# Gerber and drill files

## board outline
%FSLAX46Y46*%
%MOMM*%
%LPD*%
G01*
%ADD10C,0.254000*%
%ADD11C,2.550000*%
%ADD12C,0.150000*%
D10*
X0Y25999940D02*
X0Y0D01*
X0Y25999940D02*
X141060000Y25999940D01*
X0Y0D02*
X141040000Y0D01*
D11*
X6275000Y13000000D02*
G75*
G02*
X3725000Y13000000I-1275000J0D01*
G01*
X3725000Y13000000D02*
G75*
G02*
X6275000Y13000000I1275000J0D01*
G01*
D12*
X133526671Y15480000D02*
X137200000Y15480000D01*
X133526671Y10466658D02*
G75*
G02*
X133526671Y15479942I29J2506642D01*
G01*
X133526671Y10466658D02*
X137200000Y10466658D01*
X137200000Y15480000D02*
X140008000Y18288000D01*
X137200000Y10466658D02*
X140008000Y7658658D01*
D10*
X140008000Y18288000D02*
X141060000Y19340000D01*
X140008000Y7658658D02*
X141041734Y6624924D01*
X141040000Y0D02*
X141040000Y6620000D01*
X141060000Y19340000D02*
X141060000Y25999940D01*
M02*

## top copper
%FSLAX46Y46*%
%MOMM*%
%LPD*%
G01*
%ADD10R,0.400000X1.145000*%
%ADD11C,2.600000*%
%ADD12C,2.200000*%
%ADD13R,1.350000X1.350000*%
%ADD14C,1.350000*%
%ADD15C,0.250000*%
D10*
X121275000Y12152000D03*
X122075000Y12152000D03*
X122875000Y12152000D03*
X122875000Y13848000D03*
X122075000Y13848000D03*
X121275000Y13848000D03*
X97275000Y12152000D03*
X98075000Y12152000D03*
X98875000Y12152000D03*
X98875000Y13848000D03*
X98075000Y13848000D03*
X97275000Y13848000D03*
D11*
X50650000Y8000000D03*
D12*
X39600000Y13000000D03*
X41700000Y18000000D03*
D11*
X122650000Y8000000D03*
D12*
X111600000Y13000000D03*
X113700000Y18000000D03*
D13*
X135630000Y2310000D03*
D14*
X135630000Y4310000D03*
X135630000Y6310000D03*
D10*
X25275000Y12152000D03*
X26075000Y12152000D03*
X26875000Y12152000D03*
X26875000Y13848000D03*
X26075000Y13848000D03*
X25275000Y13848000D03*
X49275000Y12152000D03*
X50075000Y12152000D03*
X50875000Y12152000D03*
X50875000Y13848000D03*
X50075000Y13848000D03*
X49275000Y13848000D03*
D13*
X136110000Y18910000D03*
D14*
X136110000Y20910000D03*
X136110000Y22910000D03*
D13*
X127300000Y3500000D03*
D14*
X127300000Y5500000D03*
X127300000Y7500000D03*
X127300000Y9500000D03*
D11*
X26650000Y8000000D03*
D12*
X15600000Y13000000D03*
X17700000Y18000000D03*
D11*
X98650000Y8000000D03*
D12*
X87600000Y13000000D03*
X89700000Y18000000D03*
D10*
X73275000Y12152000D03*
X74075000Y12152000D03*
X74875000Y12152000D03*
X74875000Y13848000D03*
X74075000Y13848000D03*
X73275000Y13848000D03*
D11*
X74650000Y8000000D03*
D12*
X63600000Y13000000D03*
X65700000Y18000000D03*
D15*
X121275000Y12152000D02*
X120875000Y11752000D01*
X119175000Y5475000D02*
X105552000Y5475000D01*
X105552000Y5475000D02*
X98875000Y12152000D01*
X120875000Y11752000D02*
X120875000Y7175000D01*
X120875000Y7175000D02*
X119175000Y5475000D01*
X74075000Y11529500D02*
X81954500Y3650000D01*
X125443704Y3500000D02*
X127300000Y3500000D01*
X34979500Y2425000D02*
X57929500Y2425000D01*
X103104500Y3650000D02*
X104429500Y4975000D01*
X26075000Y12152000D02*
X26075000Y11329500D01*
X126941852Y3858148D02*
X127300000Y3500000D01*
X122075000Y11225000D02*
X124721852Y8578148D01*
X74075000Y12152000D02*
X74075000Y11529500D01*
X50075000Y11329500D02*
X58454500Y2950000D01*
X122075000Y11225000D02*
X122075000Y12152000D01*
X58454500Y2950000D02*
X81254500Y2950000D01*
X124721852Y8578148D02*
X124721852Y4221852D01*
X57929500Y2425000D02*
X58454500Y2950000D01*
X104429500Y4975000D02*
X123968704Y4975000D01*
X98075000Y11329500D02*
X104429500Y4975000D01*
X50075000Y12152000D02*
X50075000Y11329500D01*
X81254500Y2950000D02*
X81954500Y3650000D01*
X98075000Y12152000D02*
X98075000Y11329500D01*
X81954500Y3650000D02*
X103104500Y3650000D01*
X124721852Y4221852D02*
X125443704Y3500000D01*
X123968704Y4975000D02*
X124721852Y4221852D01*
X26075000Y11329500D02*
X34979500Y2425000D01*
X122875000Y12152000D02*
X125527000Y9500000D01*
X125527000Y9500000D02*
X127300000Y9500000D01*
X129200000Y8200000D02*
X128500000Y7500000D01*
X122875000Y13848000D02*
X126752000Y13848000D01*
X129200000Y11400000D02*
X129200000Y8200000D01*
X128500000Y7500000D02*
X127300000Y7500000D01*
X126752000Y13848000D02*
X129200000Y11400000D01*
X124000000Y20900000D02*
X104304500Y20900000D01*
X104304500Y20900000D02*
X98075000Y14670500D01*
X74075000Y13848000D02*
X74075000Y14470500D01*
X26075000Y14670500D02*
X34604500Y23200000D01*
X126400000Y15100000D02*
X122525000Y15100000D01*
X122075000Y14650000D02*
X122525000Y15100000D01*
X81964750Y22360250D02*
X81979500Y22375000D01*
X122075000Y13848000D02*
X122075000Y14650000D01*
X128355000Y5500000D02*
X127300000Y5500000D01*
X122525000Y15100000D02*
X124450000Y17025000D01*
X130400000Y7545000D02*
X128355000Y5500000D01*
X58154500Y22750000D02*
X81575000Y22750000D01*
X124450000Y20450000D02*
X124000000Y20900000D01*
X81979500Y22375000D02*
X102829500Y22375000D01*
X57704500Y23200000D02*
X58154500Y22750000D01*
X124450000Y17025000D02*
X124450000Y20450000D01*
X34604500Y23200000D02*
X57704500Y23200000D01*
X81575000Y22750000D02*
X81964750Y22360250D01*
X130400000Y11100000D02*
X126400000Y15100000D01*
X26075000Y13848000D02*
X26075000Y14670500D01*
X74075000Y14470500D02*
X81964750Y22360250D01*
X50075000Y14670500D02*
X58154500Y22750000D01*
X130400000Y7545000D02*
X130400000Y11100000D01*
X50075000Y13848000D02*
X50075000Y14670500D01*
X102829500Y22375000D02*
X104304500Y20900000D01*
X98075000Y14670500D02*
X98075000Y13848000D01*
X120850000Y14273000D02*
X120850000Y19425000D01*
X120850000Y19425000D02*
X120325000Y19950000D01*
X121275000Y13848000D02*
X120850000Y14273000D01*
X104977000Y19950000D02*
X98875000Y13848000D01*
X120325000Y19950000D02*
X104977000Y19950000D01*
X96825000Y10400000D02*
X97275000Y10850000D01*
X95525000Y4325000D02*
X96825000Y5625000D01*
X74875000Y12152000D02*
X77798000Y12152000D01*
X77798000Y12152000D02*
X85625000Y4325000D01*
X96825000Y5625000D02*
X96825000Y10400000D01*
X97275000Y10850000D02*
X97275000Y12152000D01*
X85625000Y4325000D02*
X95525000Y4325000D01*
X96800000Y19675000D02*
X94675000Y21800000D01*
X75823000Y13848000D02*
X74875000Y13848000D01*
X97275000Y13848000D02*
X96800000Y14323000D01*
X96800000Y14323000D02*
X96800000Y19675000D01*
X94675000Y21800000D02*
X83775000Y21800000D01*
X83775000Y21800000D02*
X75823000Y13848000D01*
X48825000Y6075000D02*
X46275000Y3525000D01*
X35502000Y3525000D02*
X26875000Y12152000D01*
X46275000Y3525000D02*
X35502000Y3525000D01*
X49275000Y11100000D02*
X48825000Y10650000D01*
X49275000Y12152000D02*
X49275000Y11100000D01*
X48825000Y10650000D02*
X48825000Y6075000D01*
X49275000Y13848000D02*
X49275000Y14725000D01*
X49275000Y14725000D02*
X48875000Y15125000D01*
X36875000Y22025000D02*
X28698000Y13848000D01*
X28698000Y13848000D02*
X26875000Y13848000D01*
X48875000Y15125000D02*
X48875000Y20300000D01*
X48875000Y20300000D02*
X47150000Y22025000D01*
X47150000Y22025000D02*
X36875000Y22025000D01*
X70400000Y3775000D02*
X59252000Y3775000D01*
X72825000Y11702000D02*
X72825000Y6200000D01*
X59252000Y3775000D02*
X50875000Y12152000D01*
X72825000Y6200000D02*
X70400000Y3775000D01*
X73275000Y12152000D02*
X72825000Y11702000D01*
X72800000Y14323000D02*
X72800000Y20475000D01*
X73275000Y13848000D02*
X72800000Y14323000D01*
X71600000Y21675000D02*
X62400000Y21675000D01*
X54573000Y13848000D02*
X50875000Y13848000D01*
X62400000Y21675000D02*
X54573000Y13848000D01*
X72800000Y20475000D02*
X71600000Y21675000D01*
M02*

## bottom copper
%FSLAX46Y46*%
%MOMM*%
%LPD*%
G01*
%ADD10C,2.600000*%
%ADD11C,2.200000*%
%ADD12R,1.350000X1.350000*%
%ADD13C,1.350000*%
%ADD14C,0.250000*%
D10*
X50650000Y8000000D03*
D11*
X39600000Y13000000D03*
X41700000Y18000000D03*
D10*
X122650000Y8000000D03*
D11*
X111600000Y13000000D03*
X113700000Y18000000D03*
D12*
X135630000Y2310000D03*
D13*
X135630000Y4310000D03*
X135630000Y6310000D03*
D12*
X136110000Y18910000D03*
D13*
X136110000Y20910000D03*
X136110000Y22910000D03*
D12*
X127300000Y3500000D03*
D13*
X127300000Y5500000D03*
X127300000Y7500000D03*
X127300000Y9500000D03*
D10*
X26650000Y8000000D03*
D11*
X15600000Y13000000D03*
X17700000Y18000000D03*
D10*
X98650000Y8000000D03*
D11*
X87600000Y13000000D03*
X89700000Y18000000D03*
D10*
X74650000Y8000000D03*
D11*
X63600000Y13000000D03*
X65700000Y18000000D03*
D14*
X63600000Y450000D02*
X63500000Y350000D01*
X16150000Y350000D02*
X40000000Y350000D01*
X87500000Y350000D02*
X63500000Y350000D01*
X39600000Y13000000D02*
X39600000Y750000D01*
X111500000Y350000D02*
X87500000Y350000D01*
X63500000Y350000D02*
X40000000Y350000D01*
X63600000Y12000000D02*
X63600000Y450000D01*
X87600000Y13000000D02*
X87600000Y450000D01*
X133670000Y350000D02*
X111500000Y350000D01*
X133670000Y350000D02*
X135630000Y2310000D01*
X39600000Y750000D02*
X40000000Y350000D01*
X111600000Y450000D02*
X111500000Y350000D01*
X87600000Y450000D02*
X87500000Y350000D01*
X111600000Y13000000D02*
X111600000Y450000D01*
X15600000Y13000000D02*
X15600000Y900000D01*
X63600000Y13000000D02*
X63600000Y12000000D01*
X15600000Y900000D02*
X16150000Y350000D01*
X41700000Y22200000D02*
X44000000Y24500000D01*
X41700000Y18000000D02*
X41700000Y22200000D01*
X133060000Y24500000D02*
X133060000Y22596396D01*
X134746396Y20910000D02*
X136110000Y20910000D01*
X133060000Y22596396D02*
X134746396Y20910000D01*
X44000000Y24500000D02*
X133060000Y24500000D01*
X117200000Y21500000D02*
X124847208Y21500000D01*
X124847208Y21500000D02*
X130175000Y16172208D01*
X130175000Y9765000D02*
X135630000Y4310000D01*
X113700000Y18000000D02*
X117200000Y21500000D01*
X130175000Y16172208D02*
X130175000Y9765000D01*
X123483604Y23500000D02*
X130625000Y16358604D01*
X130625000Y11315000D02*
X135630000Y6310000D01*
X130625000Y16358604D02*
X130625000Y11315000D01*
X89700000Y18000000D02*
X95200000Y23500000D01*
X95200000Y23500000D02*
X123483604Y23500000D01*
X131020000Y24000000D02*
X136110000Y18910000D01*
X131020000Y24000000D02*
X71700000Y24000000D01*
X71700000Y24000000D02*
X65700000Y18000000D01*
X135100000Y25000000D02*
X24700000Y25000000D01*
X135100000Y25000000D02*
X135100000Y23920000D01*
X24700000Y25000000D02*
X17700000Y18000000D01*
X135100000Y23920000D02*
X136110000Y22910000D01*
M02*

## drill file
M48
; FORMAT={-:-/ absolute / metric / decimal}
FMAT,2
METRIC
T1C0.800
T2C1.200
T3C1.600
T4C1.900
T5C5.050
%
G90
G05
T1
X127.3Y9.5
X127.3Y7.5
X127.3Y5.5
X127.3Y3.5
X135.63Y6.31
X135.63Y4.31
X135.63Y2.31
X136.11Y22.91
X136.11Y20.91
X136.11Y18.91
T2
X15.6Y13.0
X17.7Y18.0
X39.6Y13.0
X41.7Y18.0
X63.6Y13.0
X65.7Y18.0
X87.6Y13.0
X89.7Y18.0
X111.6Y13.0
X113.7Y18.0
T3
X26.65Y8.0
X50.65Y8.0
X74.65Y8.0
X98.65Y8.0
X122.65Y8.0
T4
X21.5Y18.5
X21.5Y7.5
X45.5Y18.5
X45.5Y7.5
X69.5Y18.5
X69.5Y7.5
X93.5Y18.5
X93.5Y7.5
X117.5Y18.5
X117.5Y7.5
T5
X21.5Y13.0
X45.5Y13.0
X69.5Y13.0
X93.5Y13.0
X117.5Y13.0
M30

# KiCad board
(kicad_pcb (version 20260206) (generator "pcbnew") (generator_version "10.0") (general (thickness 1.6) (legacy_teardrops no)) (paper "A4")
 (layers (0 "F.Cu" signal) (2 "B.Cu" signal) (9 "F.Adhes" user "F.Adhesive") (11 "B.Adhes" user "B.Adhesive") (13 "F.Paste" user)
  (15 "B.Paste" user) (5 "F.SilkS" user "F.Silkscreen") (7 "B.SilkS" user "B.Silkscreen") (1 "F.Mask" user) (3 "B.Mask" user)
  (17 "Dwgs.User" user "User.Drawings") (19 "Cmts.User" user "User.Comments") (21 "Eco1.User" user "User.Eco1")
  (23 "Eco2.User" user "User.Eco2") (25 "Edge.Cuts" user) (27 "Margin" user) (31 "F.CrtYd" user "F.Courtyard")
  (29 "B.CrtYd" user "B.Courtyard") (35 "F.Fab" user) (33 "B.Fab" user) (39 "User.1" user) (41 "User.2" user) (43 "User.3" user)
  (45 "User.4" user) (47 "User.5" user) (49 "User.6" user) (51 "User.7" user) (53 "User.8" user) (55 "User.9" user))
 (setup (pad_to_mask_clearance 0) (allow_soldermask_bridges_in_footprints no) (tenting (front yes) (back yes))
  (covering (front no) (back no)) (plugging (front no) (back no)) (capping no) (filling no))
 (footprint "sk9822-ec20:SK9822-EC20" (layer "F.Cu") (at 122.075 -13 90)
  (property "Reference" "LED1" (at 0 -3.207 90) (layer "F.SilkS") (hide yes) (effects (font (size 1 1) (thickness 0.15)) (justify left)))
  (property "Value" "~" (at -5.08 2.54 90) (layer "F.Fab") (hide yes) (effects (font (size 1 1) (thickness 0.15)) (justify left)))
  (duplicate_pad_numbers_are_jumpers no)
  (pad "1" smd rect (at -0.848 -0.8 90) (size 1.145 0.4) (layers "F.Cu" "F.Mask" "F.Paste") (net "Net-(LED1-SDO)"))
  (pad "2" smd rect (at -0.848 0 90) (size 1.145 0.4) (layers "F.Cu" "F.Mask" "F.Paste") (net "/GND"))
  (pad "3" smd rect (at -0.848 0.8 90) (size 1.145 0.4) (layers "F.Cu" "F.Mask" "F.Paste") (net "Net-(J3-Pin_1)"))
  (pad "4" smd rect (at 0.848 0.8 90) (size 1.145 0.4) (layers "F.Cu" "F.Mask" "F.Paste") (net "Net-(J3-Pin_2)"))
  (pad "5" smd rect (at 0.848 0 90) (size 1.145 0.4) (layers "F.Cu" "F.Mask" "F.Paste") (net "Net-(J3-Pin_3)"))
  (pad "6" smd rect (at 0.848 -0.8 90) (size 1.145 0.4) (layers "F.Cu" "F.Mask" "F.Paste") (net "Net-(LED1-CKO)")))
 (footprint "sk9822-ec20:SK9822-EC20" (layer "F.Cu") (at 98.075 -13 90)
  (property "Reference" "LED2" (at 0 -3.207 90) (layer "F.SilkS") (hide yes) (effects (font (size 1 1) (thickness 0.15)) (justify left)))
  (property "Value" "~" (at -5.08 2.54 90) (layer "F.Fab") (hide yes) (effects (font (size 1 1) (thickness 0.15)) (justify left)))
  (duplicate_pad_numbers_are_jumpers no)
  (pad "1" smd rect (at -0.848 -0.8 90) (size 1.145 0.4) (layers "F.Cu" "F.Mask" "F.Paste") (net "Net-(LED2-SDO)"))
  (pad "2" smd rect (at -0.848 0 90) (size 1.145 0.4) (layers "F.Cu" "F.Mask" "F.Paste") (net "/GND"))
  (pad "3" smd rect (at -0.848 0.8 90) (size 1.145 0.4) (layers "F.Cu" "F.Mask" "F.Paste") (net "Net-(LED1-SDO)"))
  (pad "4" smd rect (at 0.848 0.8 90) (size 1.145 0.4) (layers "F.Cu" "F.Mask" "F.Paste") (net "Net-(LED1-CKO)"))
  (pad "5" smd rect (at 0.848 0 90) (size 1.145 0.4) (layers "F.Cu" "F.Mask" "F.Paste") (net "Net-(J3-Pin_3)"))
  (pad "6" smd rect (at 0.848 -0.8 90) (size 1.145 0.4) (layers "F.Cu" "F.Mask" "F.Paste") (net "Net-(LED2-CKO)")))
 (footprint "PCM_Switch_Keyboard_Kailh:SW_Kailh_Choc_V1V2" (layer "F.Cu") (at 45.5 -13 90)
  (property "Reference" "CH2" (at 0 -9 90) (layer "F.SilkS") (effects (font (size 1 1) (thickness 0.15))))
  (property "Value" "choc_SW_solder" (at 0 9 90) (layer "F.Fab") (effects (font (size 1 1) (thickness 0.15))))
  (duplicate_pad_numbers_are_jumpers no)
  (pad "" np_thru_hole circle (at -5.5 0 90) (size 1.9 1.9) (drill 1.9) (layers "*.Cu" "*.Mask"))
  (pad "" thru_hole circle (at -5 5.15 90) (size 2.6 2.6) (drill 1.6) (layers "*.Cu" "*.Mask") (remove_unused_layers no)
   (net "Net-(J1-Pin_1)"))
  (pad "" np_thru_hole circle (at 0 0 90) (size 5.05 5.05) (drill 5.05) (layers "*.Cu" "*.Mask"))
  (pad "" np_thru_hole circle (at 5.5 0 90) (size 1.9 1.9) (drill 1.9) (layers "*.Cu" "*.Mask"))
  (pad "1" thru_hole circle (at 0 -5.9 90) (size 2.2 2.2) (drill 1.2) (layers "*.Cu" "*.Mask") (remove_unused_layers no)
   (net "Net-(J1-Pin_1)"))
  (pad "2" thru_hole circle (at 5 -3.8 90) (size 2.2 2.2) (drill 1.2) (layers "*.Cu" "*.Mask") (remove_unused_layers no)
   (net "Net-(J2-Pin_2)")))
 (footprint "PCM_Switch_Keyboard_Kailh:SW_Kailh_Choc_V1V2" (layer "F.Cu") (at 117.5 -13 90)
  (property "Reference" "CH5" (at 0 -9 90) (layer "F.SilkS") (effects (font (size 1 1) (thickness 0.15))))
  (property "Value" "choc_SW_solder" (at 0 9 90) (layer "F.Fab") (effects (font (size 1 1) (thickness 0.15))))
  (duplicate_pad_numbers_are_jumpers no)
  (pad "" np_thru_hole circle (at -5.5 0 90) (size 1.9 1.9) (drill 1.9) (layers "*.Cu" "*.Mask"))
  (pad "" thru_hole circle (at -5 5.15 90) (size 2.6 2.6) (drill 1.6) (layers "*.Cu" "*.Mask") (remove_unused_layers no)
   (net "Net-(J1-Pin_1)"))
  (pad "" np_thru_hole circle (at 0 0 90) (size 5.05 5.05) (drill 5.05) (layers "*.Cu" "*.Mask"))
  (pad "" np_thru_hole circle (at 5.5 0 90) (size 1.9 1.9) (drill 1.9) (layers "*.Cu" "*.Mask"))
  (pad "1" thru_hole circle (at 0 -5.9 90) (size 2.2 2.2) (drill 1.2) (layers "*.Cu" "*.Mask") (remove_unused_layers no)
   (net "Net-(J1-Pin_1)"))
  (pad "2" thru_hole circle (at 5 -3.8 90) (size 2.2 2.2) (drill 1.2) (layers "*.Cu" "*.Mask") (remove_unused_layers no)
   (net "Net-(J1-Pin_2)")))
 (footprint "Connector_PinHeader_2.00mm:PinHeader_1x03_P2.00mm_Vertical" (layer "F.Cu") (at 135.63 -2.31 180)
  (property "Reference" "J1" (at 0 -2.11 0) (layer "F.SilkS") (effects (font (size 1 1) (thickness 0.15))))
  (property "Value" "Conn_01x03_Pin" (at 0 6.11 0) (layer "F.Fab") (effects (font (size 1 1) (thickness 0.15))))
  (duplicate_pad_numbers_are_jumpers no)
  (pad "1" thru_hole rect (at 0 0 180) (size 1.35 1.35) (drill 0.8) (layers "*.Cu" "*.Mask") (remove_unused_layers no)
   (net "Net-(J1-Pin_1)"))
  (pad "2" thru_hole circle (at 0 2 180) (size 1.35 1.35) (drill 0.8) (layers "*.Cu" "*.Mask") (remove_unused_layers no)
   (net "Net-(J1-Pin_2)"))
  (pad "3" thru_hole circle (at 0 4 180) (size 1.35 1.35) (drill 0.8) (layers "*.Cu" "*.Mask") (remove_unused_layers no)
   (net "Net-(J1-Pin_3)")))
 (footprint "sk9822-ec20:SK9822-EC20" (layer "F.Cu") (at 26.075 -13 90)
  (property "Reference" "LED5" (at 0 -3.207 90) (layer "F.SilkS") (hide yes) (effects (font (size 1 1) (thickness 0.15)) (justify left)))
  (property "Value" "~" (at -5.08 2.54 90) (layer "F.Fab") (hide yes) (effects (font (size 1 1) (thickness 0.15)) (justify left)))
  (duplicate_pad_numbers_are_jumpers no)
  (pad "1" smd rect (at -0.848 -0.8 90) (size 1.145 0.4) (layers "F.Cu" "F.Mask" "F.Paste") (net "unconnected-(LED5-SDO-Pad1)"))
  (pad "2" smd rect (at -0.848 0 90) (size 1.145 0.4) (layers "F.Cu" "F.Mask" "F.Paste") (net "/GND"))
  (pad "3" smd rect (at -0.848 0.8 90) (size 1.145 0.4) (layers "F.Cu" "F.Mask" "F.Paste") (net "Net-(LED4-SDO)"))
  (pad "4" smd rect (at 0.848 0.8 90) (size 1.145 0.4) (layers "F.Cu" "F.Mask" "F.Paste") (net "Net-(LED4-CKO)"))
  (pad "5" smd rect (at 0.848 0 90) (size 1.145 0.4) (layers "F.Cu" "F.Mask" "F.Paste") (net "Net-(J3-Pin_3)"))
  (pad "6" smd rect (at 0.848 -0.8 90) (size 1.145 0.4) (layers "F.Cu" "F.Mask" "F.Paste") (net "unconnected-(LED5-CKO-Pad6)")))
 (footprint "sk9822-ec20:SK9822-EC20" (layer "F.Cu") (at 50.075 -13 90)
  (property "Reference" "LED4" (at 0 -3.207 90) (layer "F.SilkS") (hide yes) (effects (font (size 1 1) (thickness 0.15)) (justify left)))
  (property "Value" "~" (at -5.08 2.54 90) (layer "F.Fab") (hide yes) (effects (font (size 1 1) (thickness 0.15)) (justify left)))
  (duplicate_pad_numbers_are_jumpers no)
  (pad "1" smd rect (at -0.848 -0.8 90) (size 1.145 0.4) (layers "F.Cu" "F.Mask" "F.Paste") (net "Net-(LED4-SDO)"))
  (pad "2" smd rect (at -0.848 0 90) (size 1.145 0.4) (layers "F.Cu" "F.Mask" "F.Paste") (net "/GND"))
  (pad "3" smd rect (at -0.848 0.8 90) (size 1.145 0.4) (layers "F.Cu" "F.Mask" "F.Paste") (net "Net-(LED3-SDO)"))
  (pad "4" smd rect (at 0.848 0.8 90) (size 1.145 0.4) (layers "F.Cu" "F.Mask" "F.Paste") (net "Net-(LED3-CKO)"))
  (pad "5" smd rect (at 0.848 0 90) (size 1.145 0.4) (layers "F.Cu" "F.Mask" "F.Paste") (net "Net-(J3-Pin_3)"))
  (pad "6" smd rect (at 0.848 -0.8 90) (size 1.145 0.4) (layers "F.Cu" "F.Mask" "F.Paste") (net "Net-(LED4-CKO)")))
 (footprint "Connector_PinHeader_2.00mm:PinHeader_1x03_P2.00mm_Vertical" (layer "F.Cu") (at 136.11 -18.91 180)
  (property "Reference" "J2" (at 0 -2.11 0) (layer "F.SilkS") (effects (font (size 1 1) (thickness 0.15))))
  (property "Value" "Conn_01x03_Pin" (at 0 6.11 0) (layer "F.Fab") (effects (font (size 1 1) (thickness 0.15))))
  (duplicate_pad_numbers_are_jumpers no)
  (pad "1" thru_hole rect (at 0 0 180) (size 1.35 1.35) (drill 0.8) (layers "*.Cu" "*.Mask") (remove_unused_layers no)
   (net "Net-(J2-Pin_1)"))
  (pad "2" thru_hole circle (at 0 2 180) (size 1.35 1.35) (drill 0.8) (layers "*.Cu" "*.Mask") (remove_unused_layers no)
   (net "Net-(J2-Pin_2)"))
  (pad "3" thru_hole circle (at 0 4 180) (size 1.35 1.35) (drill 0.8) (layers "*.Cu" "*.Mask") (remove_unused_layers no)
   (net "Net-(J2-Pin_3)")))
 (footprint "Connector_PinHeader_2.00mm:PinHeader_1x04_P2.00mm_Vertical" (layer "F.Cu") (at 127.3 -3.5 180)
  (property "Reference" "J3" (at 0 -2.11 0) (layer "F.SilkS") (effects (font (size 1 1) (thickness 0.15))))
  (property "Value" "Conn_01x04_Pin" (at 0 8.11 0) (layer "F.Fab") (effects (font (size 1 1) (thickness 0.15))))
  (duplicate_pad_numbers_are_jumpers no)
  (pad "1" thru_hole rect (at 0 0 180) (size 1.35 1.35) (drill 0.8) (layers "*.Cu" "*.Mask") (remove_unused_layers no) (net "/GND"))
  (pad "2" thru_hole circle (at 0 2 180) (size 1.35 1.35) (drill 0.8) (layers "*.Cu" "*.Mask") (remove_unused_layers no)
   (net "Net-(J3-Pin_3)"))
  (pad "3" thru_hole circle (at 0 4 180) (size 1.35 1.35) (drill 0.8) (layers "*.Cu" "*.Mask") (remove_unused_layers no)
   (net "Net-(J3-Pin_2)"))
  (pad "4" thru_hole circle (at 0 6 180) (size 1.35 1.35) (drill 0.8) (layers "*.Cu" "*.Mask") (remove_unused_layers no)
   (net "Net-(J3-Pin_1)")))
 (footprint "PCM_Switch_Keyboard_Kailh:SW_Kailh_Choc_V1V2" (layer "F.Cu") (at 21.5 -13 90)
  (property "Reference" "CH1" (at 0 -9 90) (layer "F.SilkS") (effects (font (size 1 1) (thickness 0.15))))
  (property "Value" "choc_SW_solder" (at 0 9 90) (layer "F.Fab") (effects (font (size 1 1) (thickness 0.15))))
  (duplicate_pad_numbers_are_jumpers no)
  (pad "" np_thru_hole circle (at -5.5 0 90) (size 1.9 1.9) (drill 1.9) (layers "*.Cu" "*.Mask"))
  (pad "" thru_hole circle (at -5 5.15 90) (size 2.6 2.6) (drill 1.6) (layers "*.Cu" "*.Mask") (remove_unused_layers no)
   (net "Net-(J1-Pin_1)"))
  (pad "" np_thru_hole circle (at 0 0 90) (size 5.05 5.05) (drill 5.05) (layers "*.Cu" "*.Mask"))
  (pad "" np_thru_hole circle (at 5.5 0 90) (size 1.9 1.9) (drill 1.9) (layers "*.Cu" "*.Mask"))
  (pad "1" thru_hole circle (at 0 -5.9 90) (size 2.2 2.2) (drill 1.2) (layers "*.Cu" "*.Mask") (remove_unused_layers no)
   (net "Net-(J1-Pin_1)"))
  (pad "2" thru_hole circle (at 5 -3.8 90) (size 2.2 2.2) (drill 1.2) (layers "*.Cu" "*.Mask") (remove_unused_layers no)
   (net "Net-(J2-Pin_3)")))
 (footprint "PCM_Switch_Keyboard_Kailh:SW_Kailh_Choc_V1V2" (layer "F.Cu") (at 93.5 -13 90)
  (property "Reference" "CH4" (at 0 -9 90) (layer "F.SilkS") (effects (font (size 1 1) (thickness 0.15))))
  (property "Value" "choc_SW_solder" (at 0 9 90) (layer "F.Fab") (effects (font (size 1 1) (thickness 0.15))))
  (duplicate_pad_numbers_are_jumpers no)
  (pad "" np_thru_hole circle (at -5.5 0 90) (size 1.9 1.9) (drill 1.9) (layers "*.Cu" "*.Mask"))
  (pad "" thru_hole circle (at -5 5.15 90) (size 2.6 2.6) (drill 1.6) (layers "*.Cu" "*.Mask") (remove_unused_layers no)
   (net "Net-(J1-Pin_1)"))
  (pad "" np_thru_hole circle (at 0 0 90) (size 5.05 5.05) (drill 5.05) (layers "*.Cu" "*.Mask"))
  (pad "" np_thru_hole circle (at 5.5 0 90) (size 1.9 1.9) (drill 1.9) (layers "*.Cu" "*.Mask"))
  (pad "1" thru_hole circle (at 0 -5.9 90) (size 2.2 2.2) (drill 1.2) (layers "*.Cu" "*.Mask") (remove_unused_layers no)
   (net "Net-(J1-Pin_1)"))
  (pad "2" thru_hole circle (at 5 -3.8 90) (size 2.2 2.2) (drill 1.2) (layers "*.Cu" "*.Mask") (remove_unused_layers no)
   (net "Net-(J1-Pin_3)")))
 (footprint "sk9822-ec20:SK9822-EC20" (layer "F.Cu") (at 74.075 -13 90)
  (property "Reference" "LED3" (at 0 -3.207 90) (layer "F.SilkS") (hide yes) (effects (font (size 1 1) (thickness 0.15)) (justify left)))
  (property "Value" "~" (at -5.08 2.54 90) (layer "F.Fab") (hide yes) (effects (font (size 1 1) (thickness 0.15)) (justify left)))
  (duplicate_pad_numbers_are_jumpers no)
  (pad "1" smd rect (at -0.848 -0.8 90) (size 1.145 0.4) (layers "F.Cu" "F.Mask" "F.Paste") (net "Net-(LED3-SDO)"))
  (pad "2" smd rect (at -0.848 0 90) (size 1.145 0.4) (layers "F.Cu" "F.Mask" "F.Paste") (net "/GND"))
  (pad "3" smd rect (at -0.848 0.8 90) (size 1.145 0.4) (layers "F.Cu" "F.Mask" "F.Paste") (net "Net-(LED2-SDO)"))
  (pad "4" smd rect (at 0.848 0.8 90) (size 1.145 0.4) (layers "F.Cu" "F.Mask" "F.Paste") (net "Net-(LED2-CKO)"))
  (pad "5" smd rect (at 0.848 0 90) (size 1.145 0.4) (layers "F.Cu" "F.Mask" "F.Paste") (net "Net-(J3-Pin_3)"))
  (pad "6" smd rect (at 0.848 -0.8 90) (size 1.145 0.4) (layers "F.Cu" "F.Mask" "F.Paste") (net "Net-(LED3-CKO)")))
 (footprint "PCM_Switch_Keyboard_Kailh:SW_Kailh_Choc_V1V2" (layer "F.Cu") (at 69.5 -13 90)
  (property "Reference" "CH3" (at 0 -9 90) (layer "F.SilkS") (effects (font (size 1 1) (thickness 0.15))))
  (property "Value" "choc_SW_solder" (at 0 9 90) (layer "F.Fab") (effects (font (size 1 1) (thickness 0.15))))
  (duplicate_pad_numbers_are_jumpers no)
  (pad "" np_thru_hole circle (at -5.5 0 90) (size 1.9 1.9) (drill 1.9) (layers "*.Cu" "*.Mask"))
  (pad "" thru_hole circle (at -5 5.15 90) (size 2.6 2.6) (drill 1.6) (layers "*.Cu" "*.Mask") (remove_unused_layers no)
   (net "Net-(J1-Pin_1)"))
  (pad "" np_thru_hole circle (at 0 0 90) (size 5.05 5.05) (drill 5.05) (layers "*.Cu" "*.Mask"))
  (pad "" np_thru_hole circle (at 5.5 0 90) (size 1.9 1.9) (drill 1.9) (layers "*.Cu" "*.Mask"))
  (pad "1" thru_hole circle (at 0 -5.9 90) (size 2.2 2.2) (drill 1.2) (layers "*.Cu" "*.Mask") (remove_unused_layers no)
   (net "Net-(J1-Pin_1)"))
  (pad "2" thru_hole circle (at 5 -3.8 90) (size 2.2 2.2) (drill 1.2) (layers "*.Cu" "*.Mask") (remove_unused_layers no)
   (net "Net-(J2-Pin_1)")))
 (gr_line (start 0 -25.99994) (end 0 0) (stroke (width 0.254) (type solid)) (layer "Edge.Cuts"))
 (gr_line (start 0 -25.99994) (end 141.06 -25.99994) (stroke (width 0.254) (type solid)) (layer "Edge.Cuts"))
 (gr_line (start 0 0) (end 141.04 0) (stroke (width 0.254) (type solid)) (layer "Edge.Cuts"))
 (gr_circle (center 5 -13) (end 7.5 -13) (stroke (width 0.1) (type solid)) (fill yes) (layer "Edge.Cuts"))
 (gr_line (start 133.526671 -15.48) (end 137.2 -15.48) (stroke (width 0.15) (type default)) (layer "Edge.Cuts"))
 (gr_arc (start 133.526671 -10.466658) (mid 131.020058 -12.9733) (end 133.526671 -15.48) (stroke (width 0.15) (type default))
  (layer "Edge.Cuts"))
 (gr_line (start 133.526671 -10.466658) (end 137.2 -10.466658) (stroke (width 0.15) (type default)) (layer "Edge.Cuts"))
 (gr_line (start 137.2 -15.48) (end 140.008 -18.288) (stroke (width 0.15) (type default)) (layer "Edge.Cuts"))
 (gr_line (start 137.2 -10.466658) (end 140.008 -7.658658) (stroke (width 0.15) (type default)) (layer "Edge.Cuts"))
 (gr_line (start 140.008 -18.288) (end 141.06 -19.34) (stroke (width 0.254) (type solid)) (layer "Edge.Cuts"))
 (gr_line (start 140.008 -7.658658) (end 141.041734 -6.624924) (stroke (width 0.254) (type solid)) (layer "Edge.Cuts"))
 (gr_line (start 141.04 0) (end 141.04 -6.62) (stroke (width 0.254) (type solid)) (layer "Edge.Cuts"))
 (gr_line (start 141.06 -19.34) (end 141.06 -25.99994) (stroke (width 0.254) (type solid)) (layer "Edge.Cuts"))
 (segment (start 121.275 -12.152) (end 120.875 -11.752) (width 0.25) (layer "F.Cu") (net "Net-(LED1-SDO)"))
 (segment (start 119.175 -5.475) (end 105.552 -5.475) (width 0.25) (layer "F.Cu") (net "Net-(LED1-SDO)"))
 (segment (start 105.552 -5.475) (end 98.875 -12.152) (width 0.25) (layer "F.Cu") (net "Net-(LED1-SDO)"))
 (segment (start 120.875 -11.752) (end 120.875 -7.175) (width 0.25) (layer "F.Cu") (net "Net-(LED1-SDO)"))
 (segment (start 120.875 -7.175) (end 119.175 -5.475) (width 0.25) (layer "F.Cu") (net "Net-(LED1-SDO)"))
 (segment (start 74.075 -11.5295) (end 81.9545 -3.65) (width 0.25) (layer "F.Cu") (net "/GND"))
 (segment (start 125.443704 -3.5) (end 127.3 -3.5) (width 0.25) (layer "F.Cu") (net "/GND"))
 (segment (start 34.9795 -2.425) (end 57.9295 -2.425) (width 0.25) (layer "F.Cu") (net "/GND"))
 (segment (start 103.1045 -3.65) (end 104.4295 -4.975) (width 0.25) (layer "F.Cu") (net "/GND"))
 (segment (start 26.075 -12.152) (end 26.075 -11.3295) (width 0.25) (layer "F.Cu") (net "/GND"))
 (segment (start 126.941852 -3.858148) (end 127.3 -3.5) (width 0.25) (layer "F.Cu") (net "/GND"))
 (segment (start 122.075 -11.225) (end 124.721852 -8.578148) (width 0.25) (layer "F.Cu") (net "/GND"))
 (segment (start 74.075 -12.152) (end 74.075 -11.5295) (width 0.25) (layer "F.Cu") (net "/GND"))
 (segment (start 50.075 -11.3295) (end 58.4545 -2.95) (width 0.25) (layer "F.Cu") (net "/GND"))
 (segment (start 122.075 -11.225) (end 122.075 -12.152) (width 0.25) (layer "F.Cu") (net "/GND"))
 (segment (start 58.4545 -2.95) (end 81.2545 -2.95) (width 0.25) (layer "F.Cu") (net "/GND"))
 (segment (start 124.721852 -8.578148) (end 124.721852 -4.221852) (width 0.25) (layer "F.Cu") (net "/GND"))
 (segment (start 57.9295 -2.425) (end 58.4545 -2.95) (width 0.25) (layer "F.Cu") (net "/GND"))
 (segment (start 104.4295 -4.975) (end 123.968704 -4.975) (width 0.25) (layer "F.Cu") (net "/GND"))
 (segment (start 98.075 -11.3295) (end 104.4295 -4.975) (width 0.25) (layer "F.Cu") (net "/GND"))
 (segment (start 50.075 -12.152) (end 50.075 -11.3295) (width 0.25) (layer "F.Cu") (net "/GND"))
 (segment (start 81.2545 -2.95) (end 81.9545 -3.65) (width 0.25) (layer "F.Cu") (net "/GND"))
 (segment (start 98.075 -12.152) (end 98.075 -11.3295) (width 0.25) (layer "F.Cu") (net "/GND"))
 (segment (start 81.9545 -3.65) (end 103.1045 -3.65) (width 0.25) (layer "F.Cu") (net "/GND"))
 (segment (start 124.721852 -4.221852) (end 125.443704 -3.5) (width 0.25) (layer "F.Cu") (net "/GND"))
 (segment (start 123.968704 -4.975) (end 124.721852 -4.221852) (width 0.25) (layer "F.Cu") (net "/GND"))
 (segment (start 26.075 -11.3295) (end 34.9795 -2.425) (width 0.25) (layer "F.Cu") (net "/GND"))
 (segment (start 122.875 -12.152) (end 125.527 -9.5) (width 0.25) (layer "F.Cu") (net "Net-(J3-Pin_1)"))
 (segment (start 125.527 -9.5) (end 127.3 -9.5) (width 0.25) (layer "F.Cu") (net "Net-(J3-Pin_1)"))
 (segment (start 129.2 -8.2) (end 128.5 -7.5) (width 0.25) (layer "F.Cu") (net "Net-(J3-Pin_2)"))
 (segment (start 122.875 -13.848) (end 126.752 -13.848) (width 0.25) (layer "F.Cu") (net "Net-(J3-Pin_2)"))
 (segment (start 129.2 -11.4) (end 129.2 -8.2) (width 0.25) (layer "F.Cu") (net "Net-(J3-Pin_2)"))
 (segment (start 128.5 -7.5) (end 127.3 -7.5) (width 0.25) (layer "F.Cu") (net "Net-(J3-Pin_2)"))
 (segment (start 126.752 -13.848) (end 129.2 -11.4) (width 0.25) (layer "F.Cu") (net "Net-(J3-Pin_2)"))
 (segment (start 124 -20.9) (end 104.3045 -20.9) (width 0.25) (layer "F.Cu") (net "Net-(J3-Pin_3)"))
 (segment (start 104.3045 -20.9) (end 98.075 -14.6705) (width 0.25) (layer "F.Cu") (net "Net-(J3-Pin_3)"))
 (segment (start 74.075 -13.848) (end 74.075 -14.4705) (width 0.25) (layer "F.Cu") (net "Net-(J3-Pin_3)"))
 (segment (start 26.075 -14.6705) (end 34.6045 -23.2) (width 0.25) (layer "F.Cu") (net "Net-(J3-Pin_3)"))
 (segment (start 126.4 -15.1) (end 122.525 -15.1) (width 0.25) (layer "F.Cu") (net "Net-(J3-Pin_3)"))
 (segment (start 122.075 -14.65) (end 122.525 -15.1) (width 0.25) (layer "F.Cu") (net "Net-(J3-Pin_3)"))
 (segment (start 81.96475 -22.36025) (end 81.9795 -22.375) (width 0.25) (layer "F.Cu") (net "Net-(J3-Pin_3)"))
 (segment (start 122.075 -13.848) (end 122.075 -14.65) (width 0.25) (layer "F.Cu") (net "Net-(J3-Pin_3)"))
 (segment (start 128.355 -5.5) (end 127.3 -5.5) (width 0.25) (layer "F.Cu") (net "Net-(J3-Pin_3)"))
 (segment (start 122.525 -15.1) (end 124.45 -17.025) (width 0.25) (layer "F.Cu") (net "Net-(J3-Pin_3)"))
 (segment (start 130.4 -7.545) (end 128.355 -5.5) (width 0.25) (layer "F.Cu") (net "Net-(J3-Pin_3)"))
 (segment (start 58.1545 -22.75) (end 81.575 -22.75) (width 0.25) (layer "F.Cu") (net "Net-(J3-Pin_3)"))
 (segment (start 124.45 -20.45) (end 124 -20.9) (width 0.25) (layer "F.Cu") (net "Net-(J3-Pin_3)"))
 (segment (start 81.9795 -22.375) (end 102.8295 -22.375) (width 0.25) (layer "F.Cu") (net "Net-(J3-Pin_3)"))
 (segment (start 57.7045 -23.2) (end 58.1545 -22.75) (width 0.25) (layer "F.Cu") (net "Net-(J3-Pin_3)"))
 (segment (start 124.45 -17.025) (end 124.45 -20.45) (width 0.25) (layer "F.Cu") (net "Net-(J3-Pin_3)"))
 (segment (start 34.6045 -23.2) (end 57.7045 -23.2) (width 0.25) (layer "F.Cu") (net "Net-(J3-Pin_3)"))
 (segment (start 81.575 -22.75) (end 81.96475 -22.36025) (width 0.25) (layer "F.Cu") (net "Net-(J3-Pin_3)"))
 (segment (start 130.4 -11.1) (end 126.4 -15.1) (width 0.25) (layer "F.Cu") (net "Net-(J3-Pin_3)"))
 (segment (start 26.075 -13.848) (end 26.075 -14.6705) (width 0.25) (layer "F.Cu") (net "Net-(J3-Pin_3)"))
 (segment (start 74.075 -14.4705) (end 81.96475 -22.36025) (width 0.25) (layer "F.Cu") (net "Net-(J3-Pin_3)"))
 (segment (start 50.075 -14.6705) (end 58.1545 -22.75) (width 0.25) (layer "F.Cu") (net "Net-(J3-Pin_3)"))
 (segment (start 130.4 -7.545) (end 130.4 -11.1) (width 0.25) (layer "F.Cu") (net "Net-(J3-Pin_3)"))
 (segment (start 50.075 -13.848) (end 50.075 -14.6705) (width 0.25) (layer "F.Cu") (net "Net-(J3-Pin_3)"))
 (segment (start 102.8295 -22.375) (end 104.3045 -20.9) (width 0.25) (layer "F.Cu") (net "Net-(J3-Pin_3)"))
 (segment (start 98.075 -14.6705) (end 98.075 -13.848) (width 0.25) (layer "F.Cu") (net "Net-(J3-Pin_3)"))
 (segment (start 120.85 -14.273) (end 120.85 -19.425) (width 0.25) (layer "F.Cu") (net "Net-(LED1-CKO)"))
 (segment (start 120.85 -19.425) (end 120.325 -19.95) (width 0.25) (layer "F.Cu") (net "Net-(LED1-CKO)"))
 (segment (start 121.275 -13.848) (end 120.85 -14.273) (width 0.25) (layer "F.Cu") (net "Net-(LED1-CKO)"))
 (segment (start 104.977 -19.95) (end 98.875 -13.848) (width 0.25) (layer "F.Cu") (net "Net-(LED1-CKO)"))
 (segment (start 120.325 -19.95) (end 104.977 -19.95) (width 0.25) (layer "F.Cu") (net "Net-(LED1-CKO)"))
 (segment (start 96.825 -10.4) (end 97.275 -10.85) (width 0.25) (layer "F.Cu") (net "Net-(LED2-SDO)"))
 (segment (start 95.525 -4.325) (end 96.825 -5.625) (width 0.25) (layer "F.Cu") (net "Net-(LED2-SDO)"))
 (segment (start 74.875 -12.152) (end 77.798 -12.152) (width 0.25) (layer "F.Cu") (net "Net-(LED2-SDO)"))
 (segment (start 77.798 -12.152) (end 85.625 -4.325) (width 0.25) (layer "F.Cu") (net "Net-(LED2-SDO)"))
 (segment (start 96.825 -5.625) (end 96.825 -10.4) (width 0.25) (layer "F.Cu") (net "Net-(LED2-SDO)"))
 (segment (start 97.275 -10.85) (end 97.275 -12.152) (width 0.25) (layer "F.Cu") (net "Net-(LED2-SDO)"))
 (segment (start 85.625 -4.325) (end 95.525 -4.325) (width 0.25) (layer "F.Cu") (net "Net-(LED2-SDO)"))
 (segment (start 96.8 -19.675) (end 94.675 -21.8) (width 0.25) (layer "F.Cu") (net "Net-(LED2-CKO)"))
 (segment (start 75.823 -13.848) (end 74.875 -13.848) (width 0.25) (layer "F.Cu") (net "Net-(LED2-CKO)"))
 (segment (start 97.275 -13.848) (end 96.8 -14.323) (width 0.25) (layer "F.Cu") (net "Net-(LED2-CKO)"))
 (segment (start 96.8 -14.323) (end 96.8 -19.675) (width 0.25) (layer "F.Cu") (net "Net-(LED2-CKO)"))
 (segment (start 94.675 -21.8) (end 83.775 -21.8) (width 0.25) (layer "F.Cu") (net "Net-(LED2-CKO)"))
 (segment (start 83.775 -21.8) (end 75.823 -13.848) (width 0.25) (layer "F.Cu") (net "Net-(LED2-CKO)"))
 (segment (start 63.6 -0.45) (end 63.5 -0.35) (width 0.25) (layer "B.Cu") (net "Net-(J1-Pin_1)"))
 (segment (start 16.15 -0.35) (end 40 -0.35) (width 0.25) (layer "B.Cu") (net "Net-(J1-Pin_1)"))
 (segment (start 87.5 -0.35) (end 63.5 -0.35) (width 0.25) (layer "B.Cu") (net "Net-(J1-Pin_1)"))
 (segment (start 39.6 -13) (end 39.6 -0.75) (width 0.25) (layer "B.Cu") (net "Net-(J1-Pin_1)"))
 (segment (start 111.5 -0.35) (end 87.5 -0.35) (width 0.25) (layer "B.Cu") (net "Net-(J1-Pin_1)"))
 (segment (start 63.5 -0.35) (end 40 -0.35) (width 0.25) (layer "B.Cu") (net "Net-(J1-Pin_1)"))
 (segment (start 63.6 -12) (end 63.6 -0.45) (width 0.25) (layer "B.Cu") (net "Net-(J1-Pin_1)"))
 (segment (start 87.6 -13) (end 87.6 -0.45) (width 0.25) (layer "B.Cu") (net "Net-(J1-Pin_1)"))
 (segment (start 133.67 -0.35) (end 111.5 -0.35) (width 0.25) (layer "B.Cu") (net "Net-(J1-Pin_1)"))
 (segment (start 133.67 -0.35) (end 135.63 -2.31) (width 0.25) (layer "B.Cu") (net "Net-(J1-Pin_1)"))
 (segment (start 39.6 -0.75) (end 40 -0.35) (width 0.25) (layer "B.Cu") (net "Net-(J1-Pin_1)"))
 (segment (start 111.6 -0.45) (end 111.5 -0.35) (width 0.25) (layer "B.Cu") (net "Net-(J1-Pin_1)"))
 (segment (start 87.6 -0.45) (end 87.5 -0.35) (width 0.25) (layer "B.Cu") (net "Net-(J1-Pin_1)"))
 (segment (start 111.6 -13) (end 111.6 -0.45) (width 0.25) (layer "B.Cu") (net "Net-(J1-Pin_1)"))
 (segment (start 15.6 -13) (end 15.6 -0.9) (width 0.25) (layer "B.Cu") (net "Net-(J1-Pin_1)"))
 (segment (start 63.6 -13) (end 63.6 -12) (width 0.25) (layer "B.Cu") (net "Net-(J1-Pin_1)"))
 (segment (start 15.6 -0.9) (end 16.15 -0.35) (width 0.25) (layer "B.Cu") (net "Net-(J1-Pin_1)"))
 (segment (start 41.7 -22.2) (end 44 -24.5) (width 0.25) (layer "B.Cu") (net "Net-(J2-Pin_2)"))
 (segment (start 41.7 -18) (end 41.7 -22.2) (width 0.25) (layer "B.Cu") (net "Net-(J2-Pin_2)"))
 (segment (start 133.06 -24.5) (end 133.06 -22.596396) (width 0.25) (layer "B.Cu") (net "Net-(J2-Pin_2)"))
 (segment (start 134.746396 -20.91) (end 136.11 -20.91) (width 0.25) (layer "B.Cu") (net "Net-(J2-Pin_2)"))
 (segment (start 133.06 -22.596396) (end 134.746396 -20.91) (width 0.25) (layer "B.Cu") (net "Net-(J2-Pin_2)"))
 (segment (start 44 -24.5) (end 133.06 -24.5) (width 0.25) (layer "B.Cu") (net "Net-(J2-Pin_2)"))
 (segment (start 117.2 -21.5) (end 124.847208 -21.5) (width 0.25) (layer "B.Cu") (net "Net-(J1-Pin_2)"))
 (segment (start 124.847208 -21.5) (end 130.175 -16.172208) (width 0.25) (layer "B.Cu") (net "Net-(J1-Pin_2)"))
 (segment (start 130.175 -9.765) (end 135.63 -4.31) (width 0.25) (layer "B.Cu") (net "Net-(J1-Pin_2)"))
 (segment (start 113.7 -18) (end 117.2 -21.5) (width 0.25) (layer "B.Cu") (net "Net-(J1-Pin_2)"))
 (segment (start 130.175 -16.172208) (end 130.175 -9.765) (width 0.25) (layer "B.Cu") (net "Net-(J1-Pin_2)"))
 (segment (start 123.483604 -23.5) (end 130.625 -16.358604) (width 0.25) (layer "B.Cu") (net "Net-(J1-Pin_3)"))
 (segment (start 130.625 -11.315) (end 135.63 -6.31) (width 0.25) (layer "B.Cu") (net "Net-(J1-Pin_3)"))
 (segment (start 130.625 -16.358604) (end 130.625 -11.315) (width 0.25) (layer "B.Cu") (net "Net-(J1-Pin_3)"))
 (segment (start 89.7 -18) (end 95.2 -23.5) (width 0.25) (layer "B.Cu") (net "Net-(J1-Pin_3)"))
 (segment (start 95.2 -23.5) (end 123.483604 -23.5) (width 0.25) (layer "B.Cu") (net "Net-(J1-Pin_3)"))
 (segment (start 48.825 -6.075) (end 46.275 -3.525) (width 0.25) (layer "F.Cu") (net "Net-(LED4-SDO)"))
 (segment (start 35.502 -3.525) (end 26.875 -12.152) (width 0.25) (layer "F.Cu") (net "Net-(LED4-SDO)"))
 (segment (start 46.275 -3.525) (end 35.502 -3.525) (width 0.25) (layer "F.Cu") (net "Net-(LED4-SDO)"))
 (segment (start 49.275 -11.1) (end 48.825 -10.65) (width 0.25) (layer "F.Cu") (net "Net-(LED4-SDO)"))
 (segment (start 49.275 -12.152) (end 49.275 -11.1) (width 0.25) (layer "F.Cu") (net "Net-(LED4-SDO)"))
 (segment (start 48.825 -10.65) (end 48.825 -6.075) (width 0.25) (layer "F.Cu") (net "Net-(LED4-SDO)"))
 (segment (start 49.275 -13.848) (end 49.275 -14.725) (width 0.25) (layer "F.Cu") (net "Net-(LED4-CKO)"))
 (segment (start 49.275 -14.725) (end 48.875 -15.125) (width 0.25) (layer "F.Cu") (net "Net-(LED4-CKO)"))
 (segment (start 36.875 -22.025) (end 28.698 -13.848) (width 0.25) (layer "F.Cu") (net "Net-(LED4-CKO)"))
 (segment (start 28.698 -13.848) (end 26.875 -13.848) (width 0.25) (layer "F.Cu") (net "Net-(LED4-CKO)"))
 (segment (start 48.875 -15.125) (end 48.875 -20.3) (width 0.25) (layer "F.Cu") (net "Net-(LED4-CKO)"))
 (segment (start 48.875 -20.3) (end 47.15 -22.025) (width 0.25) (layer "F.Cu") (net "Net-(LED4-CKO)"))
 (segment (start 47.15 -22.025) (end 36.875 -22.025) (width 0.25) (layer "F.Cu") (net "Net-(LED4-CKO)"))
 (segment (start 70.4 -3.775) (end 59.252 -3.775) (width 0.25) (layer "F.Cu") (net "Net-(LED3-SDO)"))
 (segment (start 72.825 -11.702) (end 72.825 -6.2) (width 0.25) (layer "F.Cu") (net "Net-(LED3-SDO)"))
 (segment (start 59.252 -3.775) (end 50.875 -12.152) (width 0.25) (layer "F.Cu") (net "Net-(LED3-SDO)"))
 (segment (start 72.825 -6.2) (end 70.4 -3.775) (width 0.25) (layer "F.Cu") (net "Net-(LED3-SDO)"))
 (segment (start 73.275 -12.152) (end 72.825 -11.702) (width 0.25) (layer "F.Cu") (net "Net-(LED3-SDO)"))
 (segment (start 72.8 -14.323) (end 72.8 -20.475) (width 0.25) (layer "F.Cu") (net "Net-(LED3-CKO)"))
 (segment (start 73.275 -13.848) (end 72.8 -14.323) (width 0.25) (layer "F.Cu") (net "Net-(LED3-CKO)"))
 (segment (start 71.6 -21.675) (end 62.4 -21.675) (width 0.25) (layer "F.Cu") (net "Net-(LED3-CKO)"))
 (segment (start 54.573 -13.848) (end 50.875 -13.848) (width 0.25) (layer "F.Cu") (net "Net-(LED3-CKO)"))
 (segment (start 62.4 -21.675) (end 54.573 -13.848) (width 0.25) (layer "F.Cu") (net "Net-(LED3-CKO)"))
 (segment (start 72.8 -20.475) (end 71.6 -21.675) (width 0.25) (layer "F.Cu") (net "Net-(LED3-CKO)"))
 (segment (start 131.02 -24) (end 136.11 -18.91) (width 0.25) (layer "B.Cu") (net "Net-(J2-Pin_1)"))
 (segment (start 131.02 -24) (end 71.7 -24) (width 0.25) (layer "B.Cu") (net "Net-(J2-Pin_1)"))
 (segment (start 71.7 -24) (end 65.7 -18) (width 0.25) (layer "B.Cu") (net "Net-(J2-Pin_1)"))
 (segment (start 135.1 -25) (end 24.7 -25) (width 0.25) (layer "B.Cu") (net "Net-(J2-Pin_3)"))
 (segment (start 135.1 -25) (end 135.1 -23.92) (width 0.25) (layer "B.Cu") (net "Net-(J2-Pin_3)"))
 (segment (start 24.7 -25) (end 17.7 -18) (width 0.25) (layer "B.Cu") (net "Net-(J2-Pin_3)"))
 (segment (start 135.1 -23.92) (end 136.11 -22.91) (width 0.25) (layer "B.Cu") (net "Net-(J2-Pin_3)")))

